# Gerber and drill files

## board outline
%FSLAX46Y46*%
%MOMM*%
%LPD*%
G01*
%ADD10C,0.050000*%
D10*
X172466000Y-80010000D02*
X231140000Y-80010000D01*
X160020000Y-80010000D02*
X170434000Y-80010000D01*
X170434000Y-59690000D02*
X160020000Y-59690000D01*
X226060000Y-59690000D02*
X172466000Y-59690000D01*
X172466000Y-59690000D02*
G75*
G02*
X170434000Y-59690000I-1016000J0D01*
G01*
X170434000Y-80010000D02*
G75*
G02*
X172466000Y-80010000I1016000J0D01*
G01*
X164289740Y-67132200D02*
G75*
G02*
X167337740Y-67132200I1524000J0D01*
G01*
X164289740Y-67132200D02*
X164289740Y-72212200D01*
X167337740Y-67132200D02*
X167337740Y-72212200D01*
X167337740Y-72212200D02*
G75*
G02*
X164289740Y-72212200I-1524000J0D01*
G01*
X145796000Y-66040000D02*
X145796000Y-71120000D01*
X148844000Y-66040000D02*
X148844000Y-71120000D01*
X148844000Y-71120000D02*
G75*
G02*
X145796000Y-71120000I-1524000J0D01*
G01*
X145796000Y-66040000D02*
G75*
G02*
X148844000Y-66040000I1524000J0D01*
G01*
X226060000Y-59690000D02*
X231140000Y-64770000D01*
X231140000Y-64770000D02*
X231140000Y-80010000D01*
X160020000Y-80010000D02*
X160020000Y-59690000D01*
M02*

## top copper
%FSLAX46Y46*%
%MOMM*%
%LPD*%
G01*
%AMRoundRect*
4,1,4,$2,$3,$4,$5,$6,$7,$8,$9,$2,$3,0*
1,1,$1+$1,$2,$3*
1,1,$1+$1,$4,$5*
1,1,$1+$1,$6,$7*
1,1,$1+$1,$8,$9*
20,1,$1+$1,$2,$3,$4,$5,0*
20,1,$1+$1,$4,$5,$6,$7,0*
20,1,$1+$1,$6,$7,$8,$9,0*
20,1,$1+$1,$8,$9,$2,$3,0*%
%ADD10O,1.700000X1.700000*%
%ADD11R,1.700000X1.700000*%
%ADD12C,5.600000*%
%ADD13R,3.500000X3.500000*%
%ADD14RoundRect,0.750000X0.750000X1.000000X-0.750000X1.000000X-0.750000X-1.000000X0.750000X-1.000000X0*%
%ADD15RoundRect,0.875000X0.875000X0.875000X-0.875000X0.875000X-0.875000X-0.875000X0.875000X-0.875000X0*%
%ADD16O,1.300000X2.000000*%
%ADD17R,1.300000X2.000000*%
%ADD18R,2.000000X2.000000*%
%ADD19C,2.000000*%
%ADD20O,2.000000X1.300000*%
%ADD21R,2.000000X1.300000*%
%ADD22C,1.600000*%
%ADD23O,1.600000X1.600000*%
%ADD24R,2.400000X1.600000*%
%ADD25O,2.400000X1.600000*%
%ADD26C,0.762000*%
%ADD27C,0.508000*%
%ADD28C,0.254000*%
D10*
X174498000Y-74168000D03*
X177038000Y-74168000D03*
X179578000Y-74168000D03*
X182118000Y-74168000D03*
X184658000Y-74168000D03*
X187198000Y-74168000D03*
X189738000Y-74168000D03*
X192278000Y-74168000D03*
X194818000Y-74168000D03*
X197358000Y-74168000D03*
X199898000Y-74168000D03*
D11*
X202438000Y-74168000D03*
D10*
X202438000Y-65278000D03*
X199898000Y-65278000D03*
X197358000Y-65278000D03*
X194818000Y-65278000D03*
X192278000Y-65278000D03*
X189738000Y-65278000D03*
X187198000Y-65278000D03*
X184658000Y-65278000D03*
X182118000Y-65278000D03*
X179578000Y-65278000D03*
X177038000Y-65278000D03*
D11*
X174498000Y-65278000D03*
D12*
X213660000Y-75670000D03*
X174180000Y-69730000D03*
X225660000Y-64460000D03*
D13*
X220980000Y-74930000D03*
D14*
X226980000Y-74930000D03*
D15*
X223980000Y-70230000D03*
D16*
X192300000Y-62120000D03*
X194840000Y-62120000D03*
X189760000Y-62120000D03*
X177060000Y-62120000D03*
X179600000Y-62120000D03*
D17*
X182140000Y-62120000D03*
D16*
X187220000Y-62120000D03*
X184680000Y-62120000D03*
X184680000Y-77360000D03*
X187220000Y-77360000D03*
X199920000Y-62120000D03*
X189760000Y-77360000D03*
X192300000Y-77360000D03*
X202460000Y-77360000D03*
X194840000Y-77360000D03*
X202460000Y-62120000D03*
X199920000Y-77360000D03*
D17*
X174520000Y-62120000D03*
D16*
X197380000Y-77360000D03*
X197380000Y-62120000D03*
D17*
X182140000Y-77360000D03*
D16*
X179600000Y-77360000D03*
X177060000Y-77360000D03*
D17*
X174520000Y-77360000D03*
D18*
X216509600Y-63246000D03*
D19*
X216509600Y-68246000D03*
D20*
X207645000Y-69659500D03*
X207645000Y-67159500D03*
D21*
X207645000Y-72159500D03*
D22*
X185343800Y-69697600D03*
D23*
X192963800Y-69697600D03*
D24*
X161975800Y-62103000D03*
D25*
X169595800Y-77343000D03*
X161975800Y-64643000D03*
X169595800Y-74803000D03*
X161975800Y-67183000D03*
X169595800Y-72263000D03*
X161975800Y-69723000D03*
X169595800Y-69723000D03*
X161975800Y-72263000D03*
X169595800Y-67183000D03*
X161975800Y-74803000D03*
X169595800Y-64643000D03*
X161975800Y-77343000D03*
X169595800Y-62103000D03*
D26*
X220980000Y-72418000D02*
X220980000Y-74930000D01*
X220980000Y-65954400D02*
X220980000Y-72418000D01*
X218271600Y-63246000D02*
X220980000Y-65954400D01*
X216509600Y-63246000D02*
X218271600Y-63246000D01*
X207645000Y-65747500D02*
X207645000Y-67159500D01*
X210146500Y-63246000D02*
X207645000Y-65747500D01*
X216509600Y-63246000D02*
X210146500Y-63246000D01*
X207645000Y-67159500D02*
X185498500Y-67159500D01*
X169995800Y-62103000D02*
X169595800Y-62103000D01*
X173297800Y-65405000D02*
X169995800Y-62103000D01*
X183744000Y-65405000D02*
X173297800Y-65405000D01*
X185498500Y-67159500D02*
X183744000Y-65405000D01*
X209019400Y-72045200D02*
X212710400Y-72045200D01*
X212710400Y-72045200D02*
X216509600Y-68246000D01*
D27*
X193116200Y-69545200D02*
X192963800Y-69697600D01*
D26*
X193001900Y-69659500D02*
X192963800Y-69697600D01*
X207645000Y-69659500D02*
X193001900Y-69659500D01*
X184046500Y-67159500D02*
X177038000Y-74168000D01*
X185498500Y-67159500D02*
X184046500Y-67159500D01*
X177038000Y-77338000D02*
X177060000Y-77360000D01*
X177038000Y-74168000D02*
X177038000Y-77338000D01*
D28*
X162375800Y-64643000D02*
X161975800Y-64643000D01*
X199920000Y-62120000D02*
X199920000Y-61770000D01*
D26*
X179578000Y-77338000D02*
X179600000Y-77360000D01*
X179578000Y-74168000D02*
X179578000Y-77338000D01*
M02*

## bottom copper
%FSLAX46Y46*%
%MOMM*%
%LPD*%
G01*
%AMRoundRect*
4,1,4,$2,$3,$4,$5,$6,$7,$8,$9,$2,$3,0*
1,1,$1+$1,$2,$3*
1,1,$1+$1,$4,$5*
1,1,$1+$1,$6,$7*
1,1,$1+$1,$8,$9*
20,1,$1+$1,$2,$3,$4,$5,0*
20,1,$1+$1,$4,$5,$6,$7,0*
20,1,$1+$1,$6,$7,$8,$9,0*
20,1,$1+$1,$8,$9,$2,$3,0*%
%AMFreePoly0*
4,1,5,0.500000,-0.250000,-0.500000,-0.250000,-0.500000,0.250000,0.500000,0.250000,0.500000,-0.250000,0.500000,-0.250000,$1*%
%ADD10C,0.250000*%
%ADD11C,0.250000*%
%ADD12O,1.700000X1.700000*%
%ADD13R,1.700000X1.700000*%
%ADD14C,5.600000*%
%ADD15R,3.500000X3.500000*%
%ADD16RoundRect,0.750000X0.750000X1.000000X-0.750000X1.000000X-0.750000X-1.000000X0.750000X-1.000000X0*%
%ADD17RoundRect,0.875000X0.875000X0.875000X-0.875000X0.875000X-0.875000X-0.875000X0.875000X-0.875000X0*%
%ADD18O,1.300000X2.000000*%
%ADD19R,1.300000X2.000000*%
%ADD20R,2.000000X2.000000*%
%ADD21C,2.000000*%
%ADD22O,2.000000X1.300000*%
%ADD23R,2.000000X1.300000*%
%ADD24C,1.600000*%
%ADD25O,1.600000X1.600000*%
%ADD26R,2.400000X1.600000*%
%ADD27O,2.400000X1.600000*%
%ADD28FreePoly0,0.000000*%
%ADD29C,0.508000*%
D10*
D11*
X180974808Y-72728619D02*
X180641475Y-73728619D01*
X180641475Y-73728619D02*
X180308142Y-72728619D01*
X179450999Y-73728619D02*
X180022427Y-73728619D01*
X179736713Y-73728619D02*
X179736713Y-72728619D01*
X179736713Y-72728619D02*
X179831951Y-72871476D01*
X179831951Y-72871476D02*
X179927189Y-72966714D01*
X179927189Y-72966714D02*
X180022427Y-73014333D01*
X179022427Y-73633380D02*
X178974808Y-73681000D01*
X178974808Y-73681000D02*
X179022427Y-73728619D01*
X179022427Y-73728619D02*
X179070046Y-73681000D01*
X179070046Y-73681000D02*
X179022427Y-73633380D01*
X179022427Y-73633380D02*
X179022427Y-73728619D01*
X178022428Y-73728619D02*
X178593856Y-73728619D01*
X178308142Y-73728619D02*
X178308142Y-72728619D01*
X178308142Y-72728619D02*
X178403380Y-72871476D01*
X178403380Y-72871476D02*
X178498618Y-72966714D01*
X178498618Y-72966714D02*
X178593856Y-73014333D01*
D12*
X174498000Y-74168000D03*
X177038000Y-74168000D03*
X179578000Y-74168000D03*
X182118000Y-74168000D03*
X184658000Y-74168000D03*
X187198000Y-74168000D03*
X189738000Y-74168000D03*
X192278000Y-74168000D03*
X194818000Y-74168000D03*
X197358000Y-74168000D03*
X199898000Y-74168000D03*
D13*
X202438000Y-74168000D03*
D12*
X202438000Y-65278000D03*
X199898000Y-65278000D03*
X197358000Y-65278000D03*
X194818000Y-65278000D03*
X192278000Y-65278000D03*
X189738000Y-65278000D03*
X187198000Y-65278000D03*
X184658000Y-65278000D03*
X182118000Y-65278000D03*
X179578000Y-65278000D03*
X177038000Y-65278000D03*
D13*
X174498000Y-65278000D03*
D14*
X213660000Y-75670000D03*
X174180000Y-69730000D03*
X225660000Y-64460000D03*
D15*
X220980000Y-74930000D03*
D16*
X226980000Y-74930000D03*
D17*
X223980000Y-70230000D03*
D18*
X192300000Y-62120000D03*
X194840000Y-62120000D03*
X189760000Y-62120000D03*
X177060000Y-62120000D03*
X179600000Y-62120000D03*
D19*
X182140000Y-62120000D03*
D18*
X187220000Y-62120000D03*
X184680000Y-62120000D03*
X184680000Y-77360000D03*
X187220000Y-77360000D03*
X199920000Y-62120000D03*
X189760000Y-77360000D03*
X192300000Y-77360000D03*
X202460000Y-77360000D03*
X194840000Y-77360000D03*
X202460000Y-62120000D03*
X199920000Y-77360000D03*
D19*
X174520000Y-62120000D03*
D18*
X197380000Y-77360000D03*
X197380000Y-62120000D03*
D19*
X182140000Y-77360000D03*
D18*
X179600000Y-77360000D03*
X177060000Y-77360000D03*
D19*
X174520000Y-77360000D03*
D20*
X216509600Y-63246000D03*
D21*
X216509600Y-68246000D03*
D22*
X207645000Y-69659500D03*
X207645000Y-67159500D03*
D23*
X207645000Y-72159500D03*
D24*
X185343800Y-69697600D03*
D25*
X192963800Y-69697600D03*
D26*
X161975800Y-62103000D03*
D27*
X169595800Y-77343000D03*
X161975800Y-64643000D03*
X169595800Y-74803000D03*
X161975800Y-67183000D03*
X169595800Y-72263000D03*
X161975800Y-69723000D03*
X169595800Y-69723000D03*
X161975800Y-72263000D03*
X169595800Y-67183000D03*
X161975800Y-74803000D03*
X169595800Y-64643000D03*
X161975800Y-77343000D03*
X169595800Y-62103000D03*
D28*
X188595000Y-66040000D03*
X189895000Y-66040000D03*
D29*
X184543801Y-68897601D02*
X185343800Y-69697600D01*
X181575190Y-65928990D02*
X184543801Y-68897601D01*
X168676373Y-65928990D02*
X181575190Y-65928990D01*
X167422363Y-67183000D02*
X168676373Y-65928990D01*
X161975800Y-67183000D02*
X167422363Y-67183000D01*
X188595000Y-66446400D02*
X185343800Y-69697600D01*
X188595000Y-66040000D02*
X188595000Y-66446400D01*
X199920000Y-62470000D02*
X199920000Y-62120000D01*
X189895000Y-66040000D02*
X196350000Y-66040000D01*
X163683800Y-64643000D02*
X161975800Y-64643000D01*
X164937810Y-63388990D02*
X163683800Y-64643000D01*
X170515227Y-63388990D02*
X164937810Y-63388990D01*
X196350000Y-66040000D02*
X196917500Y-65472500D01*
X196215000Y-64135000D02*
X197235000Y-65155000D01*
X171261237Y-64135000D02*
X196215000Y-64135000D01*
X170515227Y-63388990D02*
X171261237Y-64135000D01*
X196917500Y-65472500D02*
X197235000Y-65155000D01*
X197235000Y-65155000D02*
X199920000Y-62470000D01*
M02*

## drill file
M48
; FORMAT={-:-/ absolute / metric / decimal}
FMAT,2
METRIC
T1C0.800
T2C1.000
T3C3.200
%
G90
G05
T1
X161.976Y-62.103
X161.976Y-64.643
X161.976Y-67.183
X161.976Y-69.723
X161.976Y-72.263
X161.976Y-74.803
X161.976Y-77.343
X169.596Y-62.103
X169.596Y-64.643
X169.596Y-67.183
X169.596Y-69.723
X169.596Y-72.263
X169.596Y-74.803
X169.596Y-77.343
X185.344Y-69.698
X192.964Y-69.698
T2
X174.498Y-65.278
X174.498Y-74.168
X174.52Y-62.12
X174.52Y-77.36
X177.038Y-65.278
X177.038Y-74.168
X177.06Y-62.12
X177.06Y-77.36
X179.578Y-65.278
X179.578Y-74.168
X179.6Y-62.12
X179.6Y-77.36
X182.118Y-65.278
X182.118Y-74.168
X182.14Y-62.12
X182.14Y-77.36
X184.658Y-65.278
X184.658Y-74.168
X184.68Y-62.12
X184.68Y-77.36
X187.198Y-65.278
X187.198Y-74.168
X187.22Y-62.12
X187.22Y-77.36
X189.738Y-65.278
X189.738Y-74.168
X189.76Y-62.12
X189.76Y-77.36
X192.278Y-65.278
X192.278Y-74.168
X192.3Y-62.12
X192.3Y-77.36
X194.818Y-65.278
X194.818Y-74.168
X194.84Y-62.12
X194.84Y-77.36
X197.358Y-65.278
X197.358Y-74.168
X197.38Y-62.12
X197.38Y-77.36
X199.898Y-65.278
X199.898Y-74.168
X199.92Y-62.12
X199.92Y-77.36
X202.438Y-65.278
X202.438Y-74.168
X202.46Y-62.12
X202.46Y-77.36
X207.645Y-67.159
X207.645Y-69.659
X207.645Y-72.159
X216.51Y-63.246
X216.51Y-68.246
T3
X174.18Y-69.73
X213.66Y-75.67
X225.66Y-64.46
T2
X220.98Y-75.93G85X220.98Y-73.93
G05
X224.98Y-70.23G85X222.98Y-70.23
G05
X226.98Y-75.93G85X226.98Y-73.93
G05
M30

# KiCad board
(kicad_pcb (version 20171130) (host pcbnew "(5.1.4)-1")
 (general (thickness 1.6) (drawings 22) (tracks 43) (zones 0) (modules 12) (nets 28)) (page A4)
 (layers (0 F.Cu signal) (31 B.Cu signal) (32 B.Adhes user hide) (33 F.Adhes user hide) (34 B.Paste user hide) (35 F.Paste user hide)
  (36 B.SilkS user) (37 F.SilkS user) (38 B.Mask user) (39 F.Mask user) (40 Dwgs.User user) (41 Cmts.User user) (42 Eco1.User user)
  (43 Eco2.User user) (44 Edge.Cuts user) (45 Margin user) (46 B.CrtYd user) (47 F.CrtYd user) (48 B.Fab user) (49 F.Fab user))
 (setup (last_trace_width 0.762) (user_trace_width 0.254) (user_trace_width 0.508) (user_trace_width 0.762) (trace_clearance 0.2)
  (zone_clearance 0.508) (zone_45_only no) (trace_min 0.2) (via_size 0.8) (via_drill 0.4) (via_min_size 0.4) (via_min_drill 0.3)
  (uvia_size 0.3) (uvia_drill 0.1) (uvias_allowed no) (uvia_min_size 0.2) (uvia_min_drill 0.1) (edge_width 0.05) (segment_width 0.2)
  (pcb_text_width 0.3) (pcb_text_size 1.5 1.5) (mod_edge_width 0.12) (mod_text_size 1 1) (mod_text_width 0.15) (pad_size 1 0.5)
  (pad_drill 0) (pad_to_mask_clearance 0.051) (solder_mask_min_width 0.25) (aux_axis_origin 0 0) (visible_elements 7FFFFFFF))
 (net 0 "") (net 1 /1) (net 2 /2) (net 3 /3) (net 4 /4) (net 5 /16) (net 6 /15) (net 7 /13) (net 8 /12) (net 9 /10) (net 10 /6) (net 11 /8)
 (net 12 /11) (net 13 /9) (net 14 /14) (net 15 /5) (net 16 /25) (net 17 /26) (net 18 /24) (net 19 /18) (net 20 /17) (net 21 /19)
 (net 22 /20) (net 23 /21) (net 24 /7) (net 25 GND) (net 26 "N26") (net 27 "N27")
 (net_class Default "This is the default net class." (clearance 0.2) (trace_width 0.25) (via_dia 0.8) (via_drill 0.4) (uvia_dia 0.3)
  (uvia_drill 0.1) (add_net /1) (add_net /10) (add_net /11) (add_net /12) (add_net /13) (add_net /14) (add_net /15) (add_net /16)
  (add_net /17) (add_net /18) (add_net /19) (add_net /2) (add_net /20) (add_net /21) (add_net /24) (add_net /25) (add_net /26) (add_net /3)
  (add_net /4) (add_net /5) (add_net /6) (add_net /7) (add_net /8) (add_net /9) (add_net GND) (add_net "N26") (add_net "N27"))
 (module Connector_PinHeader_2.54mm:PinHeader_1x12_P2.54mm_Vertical (layer F.Cu) (at 202.438 74.168 270)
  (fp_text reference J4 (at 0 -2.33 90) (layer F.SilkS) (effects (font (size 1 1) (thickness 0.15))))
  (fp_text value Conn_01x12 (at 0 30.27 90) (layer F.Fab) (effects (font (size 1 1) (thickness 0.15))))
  (pad 12 thru_hole oval (at 0 27.94 270) (size 1.7 1.7) (drill 1) (layers *.Cu *.Mask) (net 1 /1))
  (pad 11 thru_hole oval (at 0 25.4 270) (size 1.7 1.7) (drill 1) (layers *.Cu *.Mask) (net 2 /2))
  (pad 10 thru_hole oval (at 0 22.86 270) (size 1.7 1.7) (drill 1) (layers *.Cu *.Mask) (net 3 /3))
  (pad 9 thru_hole oval (at 0 20.32 270) (size 1.7 1.7) (drill 1) (layers *.Cu *.Mask) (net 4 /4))
  (pad 8 thru_hole oval (at 0 17.78 270) (size 1.7 1.7) (drill 1) (layers *.Cu *.Mask) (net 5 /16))
  (pad 7 thru_hole oval (at 0 15.24 270) (size 1.7 1.7) (drill 1) (layers *.Cu *.Mask) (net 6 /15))
  (pad 6 thru_hole oval (at 0 12.7 270) (size 1.7 1.7) (drill 1) (layers *.Cu *.Mask) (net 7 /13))
  (pad 5 thru_hole oval (at 0 10.16 270) (size 1.7 1.7) (drill 1) (layers *.Cu *.Mask) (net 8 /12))
  (pad 4 thru_hole oval (at 0 7.62 270) (size 1.7 1.7) (drill 1) (layers *.Cu *.Mask) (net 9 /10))
  (pad 3 thru_hole oval (at 0 5.08 270) (size 1.7 1.7) (drill 1) (layers *.Cu *.Mask) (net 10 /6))
  (pad 2 thru_hole oval (at 0 2.54 270) (size 1.7 1.7) (drill 1) (layers *.Cu *.Mask) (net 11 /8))
  (pad 1 thru_hole rect (at 0 0 270) (size 1.7 1.7) (drill 1) (layers *.Cu *.Mask) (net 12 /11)))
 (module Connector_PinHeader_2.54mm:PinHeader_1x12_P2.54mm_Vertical (layer F.Cu) (at 174.498 65.278 90)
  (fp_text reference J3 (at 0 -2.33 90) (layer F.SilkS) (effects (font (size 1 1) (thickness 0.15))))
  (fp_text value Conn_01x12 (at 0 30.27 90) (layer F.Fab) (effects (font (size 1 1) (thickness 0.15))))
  (pad 12 thru_hole oval (at 0 27.94 90) (size 1.7 1.7) (drill 1) (layers *.Cu *.Mask) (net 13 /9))
  (pad 11 thru_hole oval (at 0 25.4 90) (size 1.7 1.7) (drill 1) (layers *.Cu *.Mask) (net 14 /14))
  (pad 10 thru_hole oval (at 0 22.86 90) (size 1.7 1.7) (drill 1) (layers *.Cu *.Mask) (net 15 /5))
  (pad 9 thru_hole oval (at 0 20.32 90) (size 1.7 1.7) (drill 1) (layers *.Cu *.Mask) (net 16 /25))
  (pad 8 thru_hole oval (at 0 17.78 90) (size 1.7 1.7) (drill 1) (layers *.Cu *.Mask) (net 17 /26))
  (pad 7 thru_hole oval (at 0 15.24 90) (size 1.7 1.7) (drill 1) (layers *.Cu *.Mask) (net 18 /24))
  (pad 6 thru_hole oval (at 0 12.7 90) (size 1.7 1.7) (drill 1) (layers *.Cu *.Mask) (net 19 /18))
  (pad 5 thru_hole oval (at 0 10.16 90) (size 1.7 1.7) (drill 1) (layers *.Cu *.Mask) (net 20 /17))
  (pad 4 thru_hole oval (at 0 7.62 90) (size 1.7 1.7) (drill 1) (layers *.Cu *.Mask) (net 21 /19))
  (pad 3 thru_hole oval (at 0 5.08 90) (size 1.7 1.7) (drill 1) (layers *.Cu *.Mask) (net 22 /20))
  (pad 2 thru_hole oval (at 0 2.54 90) (size 1.7 1.7) (drill 1) (layers *.Cu *.Mask) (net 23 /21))
  (pad 1 thru_hole rect (at 0 0 90) (size 1.7 1.7) (drill 1) (layers *.Cu *.Mask) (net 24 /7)))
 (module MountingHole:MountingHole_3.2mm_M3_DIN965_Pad (layer F.Cu) (at 213.66 75.67)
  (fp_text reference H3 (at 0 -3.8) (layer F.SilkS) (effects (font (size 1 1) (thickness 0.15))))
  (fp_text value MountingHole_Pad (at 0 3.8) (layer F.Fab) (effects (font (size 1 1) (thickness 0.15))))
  (pad 1 thru_hole circle (at 0 0) (size 5.6 5.6) (drill 3.2) (layers *.Cu *.Mask) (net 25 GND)))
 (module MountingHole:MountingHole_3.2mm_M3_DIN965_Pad (layer F.Cu) (at 174.18 69.73)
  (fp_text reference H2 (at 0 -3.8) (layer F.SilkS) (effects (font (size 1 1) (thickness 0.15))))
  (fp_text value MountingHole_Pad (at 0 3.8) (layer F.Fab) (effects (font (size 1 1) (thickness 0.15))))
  (pad 1 thru_hole circle (at 0 0) (size 5.6 5.6) (drill 3.2) (layers *.Cu *.Mask) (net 25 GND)))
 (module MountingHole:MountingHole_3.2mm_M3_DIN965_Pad (layer F.Cu) (at 225.66 64.46)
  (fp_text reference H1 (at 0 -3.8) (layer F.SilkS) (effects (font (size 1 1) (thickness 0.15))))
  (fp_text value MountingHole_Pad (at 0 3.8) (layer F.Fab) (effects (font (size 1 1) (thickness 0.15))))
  (pad 1 thru_hole circle (at 0 0) (size 5.6 5.6) (drill 3.2) (layers *.Cu *.Mask) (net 25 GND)))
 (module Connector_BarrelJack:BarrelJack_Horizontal (layer F.Cu) (at 220.98 74.93 180)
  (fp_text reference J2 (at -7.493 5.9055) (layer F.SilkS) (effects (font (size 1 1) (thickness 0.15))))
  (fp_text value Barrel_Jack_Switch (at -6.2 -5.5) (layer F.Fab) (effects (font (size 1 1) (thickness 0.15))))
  (pad 1 thru_hole rect (at 0 0 180) (size 3.5 3.5) (drill oval 1 3) (layers *.Cu *.Mask) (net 2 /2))
  (pad 2 thru_hole roundrect (at -6 0 180) (size 3 3.5) (drill oval 1 3) (layers *.Cu *.Mask) (roundrect_rratio 0.25) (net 1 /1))
  (pad 3 thru_hole roundrect (at -3 4.7 180) (size 3.5 3.5) (drill oval 3 1) (layers *.Cu *.Mask) (roundrect_rratio 0.25) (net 1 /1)))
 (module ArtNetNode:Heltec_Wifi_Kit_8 (layer F.Cu) (at 160.02 78.74)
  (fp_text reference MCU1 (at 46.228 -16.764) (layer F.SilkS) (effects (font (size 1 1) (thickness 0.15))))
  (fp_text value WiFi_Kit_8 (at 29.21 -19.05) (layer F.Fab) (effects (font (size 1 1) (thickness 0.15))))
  (pad 26 thru_hole oval (at 32.28 -16.62) (size 1.3 2) (drill 1) (layers *.Cu *.Mask) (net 17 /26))
  (pad 25 thru_hole oval (at 34.82 -16.62) (size 1.3 2) (drill 1) (layers *.Cu *.Mask) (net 16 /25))
  (pad 24 thru_hole oval (at 29.74 -16.62) (size 1.3 2) (drill 1) (layers *.Cu *.Mask) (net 18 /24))
  (pad 21 thru_hole oval (at 17.04 -16.62) (size 1.3 2) (drill 1) (layers *.Cu *.Mask) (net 23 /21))
  (pad 20 thru_hole oval (at 19.58 -16.62) (size 1.3 2) (drill 1) (layers *.Cu *.Mask) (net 22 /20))
  (pad 19 thru_hole rect (at 22.12 -16.62) (size 1.3 2) (drill 1) (layers *.Cu *.Mask) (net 21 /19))
  (pad 18 thru_hole oval (at 27.2 -16.62) (size 1.3 2) (drill 1) (layers *.Cu *.Mask) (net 19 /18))
  (pad 17 thru_hole oval (at 24.66 -16.62) (size 1.3 2) (drill 1) (layers *.Cu *.Mask) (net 20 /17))
  (pad 16 thru_hole oval (at 24.66 -1.38) (size 1.3 2) (drill 1) (layers *.Cu *.Mask) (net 5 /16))
  (pad 15 thru_hole oval (at 27.2 -1.38) (size 1.3 2) (drill 1) (layers *.Cu *.Mask) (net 6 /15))
  (pad 14 thru_hole oval (at 39.9 -16.62) (size 1.3 2) (drill 1) (layers *.Cu *.Mask) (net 14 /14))
  (pad 13 thru_hole oval (at 29.74 -1.38) (size 1.3 2) (drill 1) (layers *.Cu *.Mask) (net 7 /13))
  (pad 12 thru_hole oval (at 32.28 -1.38) (size 1.3 2) (drill 1) (layers *.Cu *.Mask) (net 8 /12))
  (pad 11 thru_hole oval (at 42.44 -1.38) (size 1.3 2) (drill 1) (layers *.Cu *.Mask) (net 12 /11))
  (pad 10 thru_hole oval (at 34.82 -1.38) (size 1.3 2) (drill 1) (layers *.Cu *.Mask) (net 9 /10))
  (pad 9 thru_hole oval (at 42.44 -16.62) (size 1.3 2) (drill 1) (layers *.Cu *.Mask) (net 13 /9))
  (pad 8 thru_hole oval (at 39.9 -1.38) (size 1.3 2) (drill 1) (layers *.Cu *.Mask) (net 11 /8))
  (pad 7 thru_hole rect (at 14.5 -16.62) (size 1.3 2) (drill 1) (layers *.Cu *.Mask) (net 24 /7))
  (pad 6 thru_hole oval (at 37.36 -1.38) (size 1.3 2) (drill 1) (layers *.Cu *.Mask) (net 10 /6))
  (pad 5 thru_hole oval (at 37.36 -16.62) (size 1.3 2) (drill 1) (layers *.Cu *.Mask) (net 15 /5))
  (pad 4 thru_hole rect (at 22.12 -1.38) (size 1.3 2) (drill 1) (layers *.Cu *.Mask) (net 4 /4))
  (pad 3 thru_hole oval (at 19.58 -1.38) (size 1.3 2) (drill 1) (layers *.Cu *.Mask) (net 3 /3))
  (pad 2 thru_hole oval (at 17.04 -1.38) (size 1.3 2) (drill 1) (layers *.Cu *.Mask) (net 2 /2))
  (pad 1 thru_hole rect (at 14.5 -1.38) (size 1.3 2) (drill 1) (layers *.Cu *.Mask) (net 1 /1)))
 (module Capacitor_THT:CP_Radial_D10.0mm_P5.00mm (layer F.Cu) (at 216.5096 63.246 270)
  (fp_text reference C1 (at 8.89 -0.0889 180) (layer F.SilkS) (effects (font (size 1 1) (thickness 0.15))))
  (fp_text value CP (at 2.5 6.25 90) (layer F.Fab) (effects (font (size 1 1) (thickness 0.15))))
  (pad 1 thru_hole rect (at 0 0 270) (size 2 2) (drill 1) (layers *.Cu *.Mask) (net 2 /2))
  (pad 2 thru_hole circle (at 5 0 270) (size 2 2) (drill 1) (layers *.Cu *.Mask) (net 1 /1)))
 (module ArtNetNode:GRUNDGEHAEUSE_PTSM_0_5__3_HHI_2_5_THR (layer F.Cu) (at 204.645 69.6595)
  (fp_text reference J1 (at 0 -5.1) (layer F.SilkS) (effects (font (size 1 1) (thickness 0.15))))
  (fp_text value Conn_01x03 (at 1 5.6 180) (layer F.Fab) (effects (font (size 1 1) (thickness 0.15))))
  (pad 2 thru_hole oval (at 3 0 270) (size 1.3 2) (drill 1) (layers *.Cu *.Mask) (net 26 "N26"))
  (pad 1 thru_hole oval (at 3 -2.5 270) (size 1.3 2) (drill 1) (layers *.Cu *.Mask) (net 2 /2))
  (pad 3 thru_hole rect (at 3 2.5 270) (size 1.3 2) (drill 1) (layers *.Cu *.Mask) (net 1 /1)))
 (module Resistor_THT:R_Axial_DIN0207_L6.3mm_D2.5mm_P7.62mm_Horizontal (layer F.Cu) (at 185.3438 69.6976)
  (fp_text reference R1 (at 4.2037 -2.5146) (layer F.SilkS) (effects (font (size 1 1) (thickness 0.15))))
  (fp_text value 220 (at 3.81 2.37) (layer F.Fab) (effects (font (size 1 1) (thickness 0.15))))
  (pad 1 thru_hole circle (at 0 0) (size 1.6 1.6) (drill 0.8) (layers *.Cu *.Mask) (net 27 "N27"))
  (pad 2 thru_hole oval (at 7.62 0) (size 1.6 1.6) (drill 0.8) (layers *.Cu *.Mask) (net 26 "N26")))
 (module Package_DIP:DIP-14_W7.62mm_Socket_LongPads (layer F.Cu) (at 161.9758 62.103)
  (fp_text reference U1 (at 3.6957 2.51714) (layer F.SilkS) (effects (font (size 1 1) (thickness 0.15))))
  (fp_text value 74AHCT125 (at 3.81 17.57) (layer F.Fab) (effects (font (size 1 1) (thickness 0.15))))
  (pad 1 thru_hole rect (at 0 0) (size 2.4 1.6) (drill 0.8) (layers *.Cu *.Mask) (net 1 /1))
  (pad 8 thru_hole oval (at 7.62 15.24) (size 2.4 1.6) (drill 0.8) (layers *.Cu *.Mask))
  (pad 2 thru_hole oval (at 0 2.54) (size 2.4 1.6) (drill 0.8) (layers *.Cu *.Mask) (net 14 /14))
  (pad 9 thru_hole oval (at 7.62 12.7) (size 2.4 1.6) (drill 0.8) (layers *.Cu *.Mask))
  (pad 3 thru_hole oval (at 0 5.08) (size 2.4 1.6) (drill 0.8) (layers *.Cu *.Mask) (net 27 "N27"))
  (pad 10 thru_hole oval (at 7.62 10.16) (size 2.4 1.6) (drill 0.8) (layers *.Cu *.Mask))
  (pad 4 thru_hole oval (at 0 7.62) (size 2.4 1.6) (drill 0.8) (layers *.Cu *.Mask))
  (pad 11 thru_hole oval (at 7.62 7.62) (size 2.4 1.6) (drill 0.8) (layers *.Cu *.Mask))
  (pad 5 thru_hole oval (at 0 10.16) (size 2.4 1.6) (drill 0.8) (layers *.Cu *.Mask))
  (pad 12 thru_hole oval (at 7.62 5.08) (size 2.4 1.6) (drill 0.8) (layers *.Cu *.Mask))
  (pad 6 thru_hole oval (at 0 12.7) (size 2.4 1.6) (drill 0.8) (layers *.Cu *.Mask))
  (pad 13 thru_hole oval (at 7.62 2.54) (size 2.4 1.6) (drill 0.8) (layers *.Cu *.Mask))
  (pad 7 thru_hole oval (at 0 15.24) (size 2.4 1.6) (drill 0.8) (layers *.Cu *.Mask) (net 1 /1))
  (pad 14 thru_hole oval (at 7.62 0) (size 2.4 1.6) (drill 0.8) (layers *.Cu *.Mask) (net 2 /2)))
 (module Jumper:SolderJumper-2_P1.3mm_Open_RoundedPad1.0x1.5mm (layer B.Cu) (at 189.245 66.04)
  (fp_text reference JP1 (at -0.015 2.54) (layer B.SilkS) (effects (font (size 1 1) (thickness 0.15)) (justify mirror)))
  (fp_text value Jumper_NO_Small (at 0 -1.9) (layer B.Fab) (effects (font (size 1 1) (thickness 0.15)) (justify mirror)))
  (pad 1 smd custom (at -0.65 0) (size 1 0.5) (layers B.Cu B.Mask) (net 27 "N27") (zone_connect 2)
   (options (clearance outline) (anchor rect)) (primitives))
  (pad 2 smd custom (at 0.65 0) (size 1 0.5) (layers B.Cu B.Mask) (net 14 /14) (zone_connect 2) (options (clearance outline) (anchor rect))
   (primitives)))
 (gr_line (start 172.466 80.01) (end 231.14 80.01) (layer Edge.Cuts) (width 0.05))
 (gr_line (start 160.02 80.01) (end 170.434 80.01) (layer Edge.Cuts) (width 0.05))
 (gr_line (start 170.434 59.69) (end 160.02 59.69) (layer Edge.Cuts) (width 0.05))
 (gr_line (start 226.06 59.69) (end 172.466 59.69) (layer Edge.Cuts) (width 0.05))
 (gr_arc (start 171.45 59.69) (end 170.434 59.69) (angle -180) (layer Edge.Cuts) (width 0.05))
 (gr_arc (start 171.45 80.01) (end 172.466 80.01) (angle -180) (layer Edge.Cuts) (width 0.05))
 (gr_arc (start 165.81374 67.1322) (end 167.33774 67.1322) (angle -180) (layer Edge.Cuts) (width 0.05))
 (gr_line (start 164.28974 67.1322) (end 164.28974 72.2122) (layer Edge.Cuts) (width 0.05))
 (gr_line (start 167.33774 67.1322) (end 167.33774 72.2122) (layer Edge.Cuts) (width 0.05))
 (gr_arc (start 165.81374 72.2122) (end 164.28974 72.2122) (angle -180) (layer Edge.Cuts) (width 0.05))
 (gr_line (start 145.796 66.04) (end 145.796 71.12) (layer Edge.Cuts) (width 0.05))
 (gr_line (start 148.844 66.04) (end 148.844 71.12) (layer Edge.Cuts) (width 0.05))
 (gr_arc (start 147.32 71.12) (end 145.796 71.12) (angle -180) (layer Edge.Cuts) (width 0.05))
 (gr_arc (start 147.32 66.04) (end 148.844 66.04) (angle -180) (layer Edge.Cuts) (width 0.05))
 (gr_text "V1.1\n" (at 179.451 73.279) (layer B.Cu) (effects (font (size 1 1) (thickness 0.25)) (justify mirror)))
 (gr_line (start 226.06 59.69) (end 231.14 64.77) (layer Edge.Cuts) (width 0.05))
 (gr_line (start 231.14 64.77) (end 231.14 80.01) (layer Edge.Cuts) (width 0.05))
 (gr_line (start 160.02 80.01) (end 160.02 59.69) (layer Edge.Cuts) (width 0.05))
 (segment (start 220.98 72.418) (end 220.98 74.93) (width 0.762) (layer F.Cu) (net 2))
 (segment (start 220.98 65.9544) (end 220.98 72.418) (width 0.762) (layer F.Cu) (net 2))
 (segment (start 218.2716 63.246) (end 220.98 65.9544) (width 0.762) (layer F.Cu) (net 2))
 (segment (start 216.5096 63.246) (end 218.2716 63.246) (width 0.762) (layer F.Cu) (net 2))
 (segment (start 207.645 65.7475) (end 207.645 67.1595) (width 0.762) (layer F.Cu) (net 2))
 (segment (start 210.1465 63.246) (end 207.645 65.7475) (width 0.762) (layer F.Cu) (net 2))
 (segment (start 216.5096 63.246) (end 210.1465 63.246) (width 0.762) (layer F.Cu) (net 2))
 (segment (start 207.645 67.1595) (end 185.4985 67.1595) (width 0.762) (layer F.Cu) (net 2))
 (segment (start 169.9958 62.103) (end 169.5958 62.103) (width 0.762) (layer F.Cu) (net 2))
 (segment (start 173.2978 65.405) (end 169.9958 62.103) (width 0.762) (layer F.Cu) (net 2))
 (segment (start 183.744 65.405) (end 173.2978 65.405) (width 0.762) (layer F.Cu) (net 2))
 (segment (start 185.4985 67.1595) (end 183.744 65.405) (width 0.762) (layer F.Cu) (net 2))
 (segment (start 209.0194 72.0452) (end 212.7104 72.0452) (width 0.762) (layer F.Cu) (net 1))
 (segment (start 212.7104 72.0452) (end 216.5096 68.246) (width 0.762) (layer F.Cu) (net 1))
 (segment (start 193.1162 69.5452) (end 192.9638 69.6976) (width 0.508) (layer F.Cu) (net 26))
 (segment (start 193.0019 69.6595) (end 192.9638 69.6976) (width 0.762) (layer F.Cu) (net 26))
 (segment (start 207.645 69.6595) (end 193.0019 69.6595) (width 0.762) (layer F.Cu) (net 26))
 (segment (start 184.543801 68.897601) (end 185.3438 69.6976) (width 0.508) (layer B.Cu) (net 27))
 (segment (start 181.57519 65.92899) (end 184.543801 68.897601) (width 0.508) (layer B.Cu) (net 27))
 (segment (start 168.676373 65.92899) (end 181.57519 65.92899) (width 0.508) (layer B.Cu) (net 27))
 (segment (start 167.422363 67.183) (end 168.676373 65.92899) (width 0.508) (layer B.Cu) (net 27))
 (segment (start 161.9758 67.183) (end 167.422363 67.183) (width 0.508) (layer B.Cu) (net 27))
 (segment (start 188.595 66.4464) (end 185.3438 69.6976) (width 0.508) (layer B.Cu) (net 27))
 (segment (start 188.595 66.04) (end 188.595 66.4464) (width 0.508) (layer B.Cu) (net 27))
 (segment (start 184.0465 67.1595) (end 177.038 74.168) (width 0.762) (layer F.Cu) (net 2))
 (segment (start 185.4985 67.1595) (end 184.0465 67.1595) (width 0.762) (layer F.Cu) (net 2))
 (segment (start 177.038 77.338) (end 177.06 77.36) (width 0.762) (layer F.Cu) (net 2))
 (segment (start 177.038 74.168) (end 177.038 77.338) (width 0.762) (layer F.Cu) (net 2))
 (segment (start 162.3758 64.643) (end 161.9758 64.643) (width 0.254) (layer F.Cu) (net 14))
 (segment (start 199.92 62.12) (end 199.92 61.77) (width 0.254) (layer F.Cu) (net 14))
 (segment (start 199.92 62.47) (end 199.92 62.12) (width 0.508) (layer B.Cu) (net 14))
 (segment (start 189.895 66.04) (end 196.35 66.04) (width 0.508) (layer B.Cu) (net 14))
 (segment (start 163.6838 64.643) (end 161.9758 64.643) (width 0.508) (layer B.Cu) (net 14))
 (segment (start 164.93781 63.38899) (end 163.6838 64.643) (width 0.508) (layer B.Cu) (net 14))
 (segment (start 170.515227 63.38899) (end 164.93781 63.38899) (width 0.508) (layer B.Cu) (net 14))
 (segment (start 196.35 66.04) (end 196.9175 65.4725) (width 0.508) (layer B.Cu) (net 14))
 (segment (start 196.215 64.135) (end 197.235 65.155) (width 0.508) (layer B.Cu) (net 14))
 (segment (start 171.261237 64.135) (end 196.215 64.135) (width 0.508) (layer B.Cu) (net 14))
 (segment (start 170.515227 63.38899) (end 171.261237 64.135) (width 0.508) (layer B.Cu) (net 14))
 (segment (start 196.9175 65.4725) (end 197.235 65.155) (width 0.508) (layer B.Cu) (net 14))
 (segment (start 197.235 65.155) (end 199.92 62.47) (width 0.508) (layer B.Cu) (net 14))
 (segment (start 179.578 77.338) (end 179.6 77.36) (width 0.762) (layer F.Cu) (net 3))
 (segment (start 179.578 74.168) (end 179.578 77.338) (width 0.762) (layer F.Cu) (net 3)))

